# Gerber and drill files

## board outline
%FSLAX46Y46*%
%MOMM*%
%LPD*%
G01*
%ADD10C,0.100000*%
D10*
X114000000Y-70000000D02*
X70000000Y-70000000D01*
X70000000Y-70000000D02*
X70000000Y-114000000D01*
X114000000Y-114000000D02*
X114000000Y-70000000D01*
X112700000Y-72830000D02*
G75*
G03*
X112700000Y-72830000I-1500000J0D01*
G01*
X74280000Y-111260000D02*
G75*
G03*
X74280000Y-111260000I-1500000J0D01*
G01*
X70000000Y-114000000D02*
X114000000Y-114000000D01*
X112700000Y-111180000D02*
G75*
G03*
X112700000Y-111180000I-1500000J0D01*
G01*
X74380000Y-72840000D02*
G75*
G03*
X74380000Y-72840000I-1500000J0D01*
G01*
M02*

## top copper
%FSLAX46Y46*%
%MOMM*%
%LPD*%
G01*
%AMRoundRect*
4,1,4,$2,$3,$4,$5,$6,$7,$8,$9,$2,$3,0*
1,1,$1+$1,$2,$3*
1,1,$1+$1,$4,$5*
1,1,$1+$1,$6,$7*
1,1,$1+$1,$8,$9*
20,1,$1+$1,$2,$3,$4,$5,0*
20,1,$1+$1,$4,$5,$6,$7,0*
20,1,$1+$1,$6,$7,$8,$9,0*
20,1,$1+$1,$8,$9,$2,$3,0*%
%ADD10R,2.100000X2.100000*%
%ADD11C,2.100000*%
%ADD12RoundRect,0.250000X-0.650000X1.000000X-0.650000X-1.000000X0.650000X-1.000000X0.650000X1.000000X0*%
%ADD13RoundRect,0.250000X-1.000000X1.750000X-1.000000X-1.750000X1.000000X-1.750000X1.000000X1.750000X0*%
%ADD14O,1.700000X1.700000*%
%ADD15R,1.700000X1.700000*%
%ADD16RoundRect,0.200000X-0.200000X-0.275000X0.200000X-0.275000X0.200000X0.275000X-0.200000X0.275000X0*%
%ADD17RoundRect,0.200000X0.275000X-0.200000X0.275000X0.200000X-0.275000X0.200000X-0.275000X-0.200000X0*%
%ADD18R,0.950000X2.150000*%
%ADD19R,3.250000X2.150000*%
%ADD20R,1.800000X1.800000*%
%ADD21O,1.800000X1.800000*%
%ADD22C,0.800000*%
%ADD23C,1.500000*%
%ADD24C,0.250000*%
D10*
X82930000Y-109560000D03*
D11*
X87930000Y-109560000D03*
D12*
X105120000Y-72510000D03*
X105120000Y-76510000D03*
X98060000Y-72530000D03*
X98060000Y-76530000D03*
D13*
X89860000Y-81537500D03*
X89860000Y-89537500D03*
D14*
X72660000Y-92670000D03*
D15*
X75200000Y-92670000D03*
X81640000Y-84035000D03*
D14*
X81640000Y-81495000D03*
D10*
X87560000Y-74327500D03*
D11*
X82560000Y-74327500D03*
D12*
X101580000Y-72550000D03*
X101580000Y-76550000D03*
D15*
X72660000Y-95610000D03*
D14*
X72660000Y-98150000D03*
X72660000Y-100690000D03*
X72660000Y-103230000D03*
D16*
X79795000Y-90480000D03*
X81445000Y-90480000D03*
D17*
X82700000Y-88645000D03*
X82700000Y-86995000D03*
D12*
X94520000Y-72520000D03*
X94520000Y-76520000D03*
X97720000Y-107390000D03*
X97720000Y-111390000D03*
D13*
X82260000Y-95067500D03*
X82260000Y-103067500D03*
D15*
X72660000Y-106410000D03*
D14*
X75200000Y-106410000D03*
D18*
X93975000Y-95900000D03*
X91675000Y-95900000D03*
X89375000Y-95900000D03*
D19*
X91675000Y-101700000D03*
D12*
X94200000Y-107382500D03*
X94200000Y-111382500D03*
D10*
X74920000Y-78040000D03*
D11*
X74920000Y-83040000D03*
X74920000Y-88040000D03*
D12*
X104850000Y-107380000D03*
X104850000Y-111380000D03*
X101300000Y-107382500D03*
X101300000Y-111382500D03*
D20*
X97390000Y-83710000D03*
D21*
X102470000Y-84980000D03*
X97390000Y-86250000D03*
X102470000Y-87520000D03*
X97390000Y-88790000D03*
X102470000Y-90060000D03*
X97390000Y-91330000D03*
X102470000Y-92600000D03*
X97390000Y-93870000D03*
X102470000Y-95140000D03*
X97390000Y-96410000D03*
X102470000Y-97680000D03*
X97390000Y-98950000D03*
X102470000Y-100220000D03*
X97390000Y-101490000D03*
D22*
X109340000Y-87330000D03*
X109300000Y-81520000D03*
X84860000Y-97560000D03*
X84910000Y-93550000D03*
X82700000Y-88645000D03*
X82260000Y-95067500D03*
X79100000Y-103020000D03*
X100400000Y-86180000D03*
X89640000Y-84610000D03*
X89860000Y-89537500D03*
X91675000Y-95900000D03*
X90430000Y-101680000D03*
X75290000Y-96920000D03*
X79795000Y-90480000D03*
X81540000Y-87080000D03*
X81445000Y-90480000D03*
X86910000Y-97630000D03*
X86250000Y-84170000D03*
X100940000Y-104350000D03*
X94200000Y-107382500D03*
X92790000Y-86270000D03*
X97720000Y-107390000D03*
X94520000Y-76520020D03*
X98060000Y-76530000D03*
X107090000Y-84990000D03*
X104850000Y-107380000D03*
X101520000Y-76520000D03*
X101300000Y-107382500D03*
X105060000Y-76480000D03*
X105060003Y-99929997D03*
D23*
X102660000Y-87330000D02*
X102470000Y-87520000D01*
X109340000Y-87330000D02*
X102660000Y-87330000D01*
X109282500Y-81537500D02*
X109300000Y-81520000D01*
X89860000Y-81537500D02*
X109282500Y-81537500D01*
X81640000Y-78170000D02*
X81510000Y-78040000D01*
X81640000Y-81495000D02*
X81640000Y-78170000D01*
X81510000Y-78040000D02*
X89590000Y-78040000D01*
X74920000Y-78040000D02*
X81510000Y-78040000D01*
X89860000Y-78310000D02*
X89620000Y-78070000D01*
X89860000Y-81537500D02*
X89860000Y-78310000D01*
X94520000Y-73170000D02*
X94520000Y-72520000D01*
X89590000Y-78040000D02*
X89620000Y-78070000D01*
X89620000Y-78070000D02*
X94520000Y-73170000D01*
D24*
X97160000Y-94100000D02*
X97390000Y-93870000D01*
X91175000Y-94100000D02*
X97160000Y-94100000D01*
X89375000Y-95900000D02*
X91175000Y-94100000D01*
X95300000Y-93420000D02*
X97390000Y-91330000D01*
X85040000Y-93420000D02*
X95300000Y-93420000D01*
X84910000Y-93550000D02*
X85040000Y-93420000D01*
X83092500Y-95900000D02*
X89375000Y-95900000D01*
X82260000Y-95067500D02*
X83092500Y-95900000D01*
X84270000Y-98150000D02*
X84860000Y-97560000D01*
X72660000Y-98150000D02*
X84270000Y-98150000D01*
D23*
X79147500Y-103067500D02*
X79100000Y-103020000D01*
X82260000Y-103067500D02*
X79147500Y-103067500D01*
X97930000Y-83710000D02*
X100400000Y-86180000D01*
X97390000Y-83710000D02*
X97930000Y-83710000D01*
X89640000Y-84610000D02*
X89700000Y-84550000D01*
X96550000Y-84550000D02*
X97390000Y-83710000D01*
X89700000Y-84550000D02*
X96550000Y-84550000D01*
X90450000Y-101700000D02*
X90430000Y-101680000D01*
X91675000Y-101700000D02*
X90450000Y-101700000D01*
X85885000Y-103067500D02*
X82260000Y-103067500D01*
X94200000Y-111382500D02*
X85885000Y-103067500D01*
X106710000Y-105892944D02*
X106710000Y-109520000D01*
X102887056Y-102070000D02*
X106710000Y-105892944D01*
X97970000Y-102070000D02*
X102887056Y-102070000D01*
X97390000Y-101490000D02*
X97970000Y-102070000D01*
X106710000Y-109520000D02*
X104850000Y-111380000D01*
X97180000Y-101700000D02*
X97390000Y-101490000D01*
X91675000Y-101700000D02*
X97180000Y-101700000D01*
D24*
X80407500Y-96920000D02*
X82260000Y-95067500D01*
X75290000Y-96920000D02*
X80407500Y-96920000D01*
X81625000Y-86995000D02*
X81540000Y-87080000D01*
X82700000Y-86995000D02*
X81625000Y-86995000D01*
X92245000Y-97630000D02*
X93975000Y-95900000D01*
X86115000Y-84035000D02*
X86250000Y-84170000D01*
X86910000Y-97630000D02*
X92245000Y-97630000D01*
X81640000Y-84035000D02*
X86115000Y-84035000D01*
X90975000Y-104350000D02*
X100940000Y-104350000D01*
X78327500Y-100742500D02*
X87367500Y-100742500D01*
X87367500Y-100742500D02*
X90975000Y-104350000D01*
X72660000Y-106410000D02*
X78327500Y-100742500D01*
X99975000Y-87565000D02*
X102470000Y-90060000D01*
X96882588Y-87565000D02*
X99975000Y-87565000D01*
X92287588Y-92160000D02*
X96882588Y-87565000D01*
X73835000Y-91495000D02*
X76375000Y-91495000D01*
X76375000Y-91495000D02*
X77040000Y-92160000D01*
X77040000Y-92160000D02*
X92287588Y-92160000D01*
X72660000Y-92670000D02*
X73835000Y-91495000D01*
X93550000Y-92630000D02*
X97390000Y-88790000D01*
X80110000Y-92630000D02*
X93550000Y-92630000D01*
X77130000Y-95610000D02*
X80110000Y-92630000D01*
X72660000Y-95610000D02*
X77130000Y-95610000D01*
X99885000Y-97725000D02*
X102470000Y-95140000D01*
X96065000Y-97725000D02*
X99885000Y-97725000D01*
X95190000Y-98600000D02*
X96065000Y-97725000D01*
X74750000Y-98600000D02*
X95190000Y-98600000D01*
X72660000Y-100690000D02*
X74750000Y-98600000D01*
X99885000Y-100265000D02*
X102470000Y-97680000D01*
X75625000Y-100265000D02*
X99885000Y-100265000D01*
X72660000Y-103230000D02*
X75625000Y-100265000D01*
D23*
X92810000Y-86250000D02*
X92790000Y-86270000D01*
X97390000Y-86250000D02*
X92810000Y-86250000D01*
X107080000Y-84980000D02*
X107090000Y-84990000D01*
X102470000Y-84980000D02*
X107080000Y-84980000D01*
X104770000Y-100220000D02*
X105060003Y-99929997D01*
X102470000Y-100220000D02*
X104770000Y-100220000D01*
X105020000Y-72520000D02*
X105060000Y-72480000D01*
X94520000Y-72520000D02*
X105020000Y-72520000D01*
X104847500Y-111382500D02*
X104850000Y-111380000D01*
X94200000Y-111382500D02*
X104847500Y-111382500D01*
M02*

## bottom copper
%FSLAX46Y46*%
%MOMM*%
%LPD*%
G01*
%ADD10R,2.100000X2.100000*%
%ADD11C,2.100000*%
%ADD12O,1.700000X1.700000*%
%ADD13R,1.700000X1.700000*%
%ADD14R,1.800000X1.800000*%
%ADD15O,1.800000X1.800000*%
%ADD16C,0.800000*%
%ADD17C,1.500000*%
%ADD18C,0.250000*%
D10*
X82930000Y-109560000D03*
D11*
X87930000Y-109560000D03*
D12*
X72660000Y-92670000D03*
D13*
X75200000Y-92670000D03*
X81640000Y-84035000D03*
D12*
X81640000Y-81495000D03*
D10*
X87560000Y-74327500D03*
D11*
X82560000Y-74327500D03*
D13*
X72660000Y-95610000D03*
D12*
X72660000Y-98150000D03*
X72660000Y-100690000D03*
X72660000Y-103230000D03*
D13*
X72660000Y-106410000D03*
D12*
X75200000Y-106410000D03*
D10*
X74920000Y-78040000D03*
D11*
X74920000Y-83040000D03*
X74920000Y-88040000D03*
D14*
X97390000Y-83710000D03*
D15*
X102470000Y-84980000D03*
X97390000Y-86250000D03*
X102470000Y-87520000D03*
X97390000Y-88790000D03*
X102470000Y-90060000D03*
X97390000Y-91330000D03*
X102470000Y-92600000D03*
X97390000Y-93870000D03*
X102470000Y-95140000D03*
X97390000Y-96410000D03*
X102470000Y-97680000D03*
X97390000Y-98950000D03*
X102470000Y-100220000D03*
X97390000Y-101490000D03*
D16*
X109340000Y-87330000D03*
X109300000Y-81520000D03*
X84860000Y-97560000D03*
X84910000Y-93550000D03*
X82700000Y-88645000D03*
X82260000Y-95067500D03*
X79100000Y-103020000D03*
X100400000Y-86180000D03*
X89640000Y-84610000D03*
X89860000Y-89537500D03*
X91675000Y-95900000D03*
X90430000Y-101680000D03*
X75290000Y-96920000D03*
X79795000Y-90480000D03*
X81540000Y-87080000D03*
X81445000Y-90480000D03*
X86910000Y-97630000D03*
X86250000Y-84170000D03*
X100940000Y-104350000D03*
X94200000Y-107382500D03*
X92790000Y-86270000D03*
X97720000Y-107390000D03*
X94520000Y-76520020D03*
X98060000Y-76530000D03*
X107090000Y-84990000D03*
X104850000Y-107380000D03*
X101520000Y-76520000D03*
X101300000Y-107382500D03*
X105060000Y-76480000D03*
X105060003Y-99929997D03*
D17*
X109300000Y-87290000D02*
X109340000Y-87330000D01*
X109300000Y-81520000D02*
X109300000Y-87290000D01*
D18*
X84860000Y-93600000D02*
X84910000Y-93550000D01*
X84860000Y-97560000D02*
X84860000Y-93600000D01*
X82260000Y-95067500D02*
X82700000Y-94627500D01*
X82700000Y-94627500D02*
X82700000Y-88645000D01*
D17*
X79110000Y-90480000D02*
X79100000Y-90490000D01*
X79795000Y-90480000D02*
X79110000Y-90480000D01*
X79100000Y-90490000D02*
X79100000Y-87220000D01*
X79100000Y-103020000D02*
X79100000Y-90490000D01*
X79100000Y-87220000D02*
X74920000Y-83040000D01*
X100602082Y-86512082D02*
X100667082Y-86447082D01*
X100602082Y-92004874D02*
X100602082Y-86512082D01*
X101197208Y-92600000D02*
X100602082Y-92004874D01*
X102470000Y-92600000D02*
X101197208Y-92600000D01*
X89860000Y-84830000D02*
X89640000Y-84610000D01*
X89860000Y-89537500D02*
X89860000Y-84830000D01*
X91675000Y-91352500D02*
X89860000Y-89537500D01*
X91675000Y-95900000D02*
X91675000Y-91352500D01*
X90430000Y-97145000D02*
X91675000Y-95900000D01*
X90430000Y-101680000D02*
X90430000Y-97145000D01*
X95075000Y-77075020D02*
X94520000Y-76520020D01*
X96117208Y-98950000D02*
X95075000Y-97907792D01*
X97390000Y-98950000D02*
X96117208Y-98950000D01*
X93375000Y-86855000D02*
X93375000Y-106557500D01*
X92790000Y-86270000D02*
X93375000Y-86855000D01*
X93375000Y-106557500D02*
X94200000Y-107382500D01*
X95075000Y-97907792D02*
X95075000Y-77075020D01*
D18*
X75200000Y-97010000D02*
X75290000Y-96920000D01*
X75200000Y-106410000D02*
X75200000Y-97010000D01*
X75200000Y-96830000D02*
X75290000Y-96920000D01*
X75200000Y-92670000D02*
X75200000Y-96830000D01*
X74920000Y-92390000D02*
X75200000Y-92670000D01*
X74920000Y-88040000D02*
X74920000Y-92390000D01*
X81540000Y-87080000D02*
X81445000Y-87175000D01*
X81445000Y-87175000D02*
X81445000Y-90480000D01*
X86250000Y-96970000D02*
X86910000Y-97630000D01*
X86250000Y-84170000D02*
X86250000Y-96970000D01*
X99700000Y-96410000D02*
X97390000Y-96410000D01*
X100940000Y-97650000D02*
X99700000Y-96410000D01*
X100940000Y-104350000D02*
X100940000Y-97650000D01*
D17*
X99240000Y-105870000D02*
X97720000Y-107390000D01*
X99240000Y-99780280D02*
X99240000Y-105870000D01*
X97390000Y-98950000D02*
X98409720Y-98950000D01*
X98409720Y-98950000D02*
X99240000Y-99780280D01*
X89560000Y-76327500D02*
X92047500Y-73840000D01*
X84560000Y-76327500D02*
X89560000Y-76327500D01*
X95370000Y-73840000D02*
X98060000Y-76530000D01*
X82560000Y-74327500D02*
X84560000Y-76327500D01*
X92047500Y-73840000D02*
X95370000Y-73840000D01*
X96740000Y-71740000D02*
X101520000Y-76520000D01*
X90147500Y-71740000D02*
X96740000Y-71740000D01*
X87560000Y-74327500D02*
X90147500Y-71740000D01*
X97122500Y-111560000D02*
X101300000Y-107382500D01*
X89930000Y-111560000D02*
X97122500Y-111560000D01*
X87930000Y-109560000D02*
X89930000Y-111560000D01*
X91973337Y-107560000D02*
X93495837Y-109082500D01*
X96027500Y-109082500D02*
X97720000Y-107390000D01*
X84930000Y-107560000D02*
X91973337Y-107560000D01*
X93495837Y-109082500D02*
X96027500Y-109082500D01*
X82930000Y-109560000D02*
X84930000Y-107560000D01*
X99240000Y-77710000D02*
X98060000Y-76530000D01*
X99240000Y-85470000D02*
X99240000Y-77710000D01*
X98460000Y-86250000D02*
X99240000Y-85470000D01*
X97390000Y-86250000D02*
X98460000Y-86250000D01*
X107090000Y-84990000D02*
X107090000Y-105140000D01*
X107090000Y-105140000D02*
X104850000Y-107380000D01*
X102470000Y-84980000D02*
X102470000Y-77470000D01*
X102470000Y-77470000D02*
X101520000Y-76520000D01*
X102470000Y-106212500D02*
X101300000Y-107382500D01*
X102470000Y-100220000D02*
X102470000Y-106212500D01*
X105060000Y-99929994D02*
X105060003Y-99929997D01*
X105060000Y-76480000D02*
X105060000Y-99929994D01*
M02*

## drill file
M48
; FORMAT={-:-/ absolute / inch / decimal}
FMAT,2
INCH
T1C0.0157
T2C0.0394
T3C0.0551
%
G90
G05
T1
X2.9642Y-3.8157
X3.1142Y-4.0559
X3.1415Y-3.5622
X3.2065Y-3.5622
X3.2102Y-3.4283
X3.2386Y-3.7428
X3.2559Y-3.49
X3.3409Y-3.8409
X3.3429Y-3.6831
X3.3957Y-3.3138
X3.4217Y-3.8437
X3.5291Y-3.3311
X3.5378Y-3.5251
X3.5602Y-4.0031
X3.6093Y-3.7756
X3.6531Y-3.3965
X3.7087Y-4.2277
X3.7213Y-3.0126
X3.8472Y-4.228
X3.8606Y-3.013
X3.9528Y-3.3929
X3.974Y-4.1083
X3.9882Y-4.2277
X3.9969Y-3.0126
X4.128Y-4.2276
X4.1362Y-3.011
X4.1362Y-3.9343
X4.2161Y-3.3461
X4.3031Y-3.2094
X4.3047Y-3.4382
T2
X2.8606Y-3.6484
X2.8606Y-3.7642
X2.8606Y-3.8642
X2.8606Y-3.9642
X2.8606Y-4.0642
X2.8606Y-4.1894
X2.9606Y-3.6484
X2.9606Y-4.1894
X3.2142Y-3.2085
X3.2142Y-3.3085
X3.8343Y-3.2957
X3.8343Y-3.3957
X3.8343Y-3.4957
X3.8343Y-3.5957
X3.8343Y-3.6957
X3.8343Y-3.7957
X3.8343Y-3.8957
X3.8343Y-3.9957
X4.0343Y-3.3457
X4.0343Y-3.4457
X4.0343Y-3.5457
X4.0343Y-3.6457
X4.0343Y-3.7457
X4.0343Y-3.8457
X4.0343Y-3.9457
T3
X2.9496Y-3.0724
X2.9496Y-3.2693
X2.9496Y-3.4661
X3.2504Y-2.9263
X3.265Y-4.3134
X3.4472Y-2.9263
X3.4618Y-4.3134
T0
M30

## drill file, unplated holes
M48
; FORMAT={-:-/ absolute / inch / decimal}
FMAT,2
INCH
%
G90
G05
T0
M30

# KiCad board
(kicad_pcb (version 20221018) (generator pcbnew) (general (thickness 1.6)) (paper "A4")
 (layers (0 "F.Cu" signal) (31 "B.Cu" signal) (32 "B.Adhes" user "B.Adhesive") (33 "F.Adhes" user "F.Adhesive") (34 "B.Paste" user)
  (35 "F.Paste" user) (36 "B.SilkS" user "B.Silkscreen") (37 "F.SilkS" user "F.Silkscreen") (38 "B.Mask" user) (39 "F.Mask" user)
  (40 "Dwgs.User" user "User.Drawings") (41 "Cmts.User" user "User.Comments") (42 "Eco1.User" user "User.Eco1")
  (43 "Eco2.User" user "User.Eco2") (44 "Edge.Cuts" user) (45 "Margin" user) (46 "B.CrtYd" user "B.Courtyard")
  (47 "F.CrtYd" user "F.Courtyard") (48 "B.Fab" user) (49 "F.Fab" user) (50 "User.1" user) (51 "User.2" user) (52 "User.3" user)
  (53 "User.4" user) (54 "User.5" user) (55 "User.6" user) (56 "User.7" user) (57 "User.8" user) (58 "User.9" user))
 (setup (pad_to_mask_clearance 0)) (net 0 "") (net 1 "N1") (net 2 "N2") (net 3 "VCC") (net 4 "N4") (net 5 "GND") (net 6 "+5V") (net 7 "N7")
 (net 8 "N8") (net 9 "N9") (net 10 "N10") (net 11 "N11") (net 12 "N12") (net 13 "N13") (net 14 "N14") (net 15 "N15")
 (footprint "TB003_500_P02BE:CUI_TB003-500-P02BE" (layer "F.Cu") (at 82.93 109.56)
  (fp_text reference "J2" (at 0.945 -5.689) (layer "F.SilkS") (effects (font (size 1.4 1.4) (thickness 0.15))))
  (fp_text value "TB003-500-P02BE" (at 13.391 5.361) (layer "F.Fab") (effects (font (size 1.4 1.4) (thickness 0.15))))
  (pad "1" thru_hole rect (at 0 0) (size 2.1 2.1) (drill 1.4) (layers "*.Cu" "*.Mask") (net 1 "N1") (solder_mask_margin 0.102))
  (pad "2" thru_hole circle (at 5 0) (size 2.1 2.1) (drill 1.4) (layers "*.Cu" "*.Mask") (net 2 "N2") (solder_mask_margin 0.102)))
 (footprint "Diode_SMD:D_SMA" (layer "F.Cu") (at 105.12 74.51 -90)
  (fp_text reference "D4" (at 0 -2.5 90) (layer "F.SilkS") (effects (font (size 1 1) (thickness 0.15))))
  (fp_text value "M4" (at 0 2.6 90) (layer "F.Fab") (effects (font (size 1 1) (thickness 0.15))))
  (pad "1" smd roundrect (at -2 0 270) (size 2.5 1.8) (layers "F.Cu" "F.Paste" "F.Mask") (roundrect_rratio 0.1388888889) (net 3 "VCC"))
  (pad "2" smd roundrect (at 2 0 270) (size 2.5 1.8) (layers "F.Cu" "F.Paste" "F.Mask") (roundrect_rratio 0.1388888889) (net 2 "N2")))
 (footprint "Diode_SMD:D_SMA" (layer "F.Cu") (at 98.06 74.53 -90)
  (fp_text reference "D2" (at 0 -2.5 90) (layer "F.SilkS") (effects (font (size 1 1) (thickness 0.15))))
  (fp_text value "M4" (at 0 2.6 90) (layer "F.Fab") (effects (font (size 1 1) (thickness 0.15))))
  (pad "1" smd roundrect (at -2 0 270) (size 2.5 1.8) (layers "F.Cu" "F.Paste" "F.Mask") (roundrect_rratio 0.1388888889) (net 3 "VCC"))
  (pad "2" smd roundrect (at 2 0 270) (size 2.5 1.8) (layers "F.Cu" "F.Paste" "F.Mask") (roundrect_rratio 0.1388888889) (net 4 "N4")))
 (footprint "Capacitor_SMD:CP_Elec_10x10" (layer "F.Cu") (at 89.86 85.5375 -90)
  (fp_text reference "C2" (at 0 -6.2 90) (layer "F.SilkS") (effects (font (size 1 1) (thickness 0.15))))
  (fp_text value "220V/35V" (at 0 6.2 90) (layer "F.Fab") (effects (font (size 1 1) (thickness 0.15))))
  (pad "1" smd roundrect (at -4 0 270) (size 4 2.5) (layers "F.Cu" "F.Paste" "F.Mask") (roundrect_rratio 0.1) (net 3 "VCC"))
  (pad "2" smd roundrect (at 4 0 270) (size 4 2.5) (layers "F.Cu" "F.Paste" "F.Mask") (roundrect_rratio 0.1) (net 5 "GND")))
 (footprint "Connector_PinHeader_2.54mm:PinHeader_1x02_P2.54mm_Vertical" (layer "F.Cu") (at 75.2 92.67 -90)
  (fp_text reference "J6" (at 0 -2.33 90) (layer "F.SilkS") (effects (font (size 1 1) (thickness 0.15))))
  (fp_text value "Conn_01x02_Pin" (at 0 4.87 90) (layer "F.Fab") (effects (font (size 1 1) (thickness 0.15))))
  (pad "1" thru_hole rect (at 0 0 270) (size 1.7 1.7) (drill 1) (layers "*.Cu" "*.Mask") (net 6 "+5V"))
  (pad "2" thru_hole oval (at 0 2.54 270) (size 1.7 1.7) (drill 1) (layers "*.Cu" "*.Mask") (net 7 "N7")))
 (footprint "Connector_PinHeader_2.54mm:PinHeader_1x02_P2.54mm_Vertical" (layer "F.Cu") (at 81.64 84.035 180)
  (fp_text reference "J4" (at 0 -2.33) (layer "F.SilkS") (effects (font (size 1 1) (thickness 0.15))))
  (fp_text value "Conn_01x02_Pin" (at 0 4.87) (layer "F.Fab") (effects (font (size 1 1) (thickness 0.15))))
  (pad "1" thru_hole rect (at 0 0 180) (size 1.7 1.7) (drill 1) (layers "*.Cu" "*.Mask") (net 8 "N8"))
  (pad "2" thru_hole oval (at 0 2.54 180) (size 1.7 1.7) (drill 1) (layers "*.Cu" "*.Mask") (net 3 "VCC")))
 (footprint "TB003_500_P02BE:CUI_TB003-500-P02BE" (layer "F.Cu") (at 87.56 74.3275 180)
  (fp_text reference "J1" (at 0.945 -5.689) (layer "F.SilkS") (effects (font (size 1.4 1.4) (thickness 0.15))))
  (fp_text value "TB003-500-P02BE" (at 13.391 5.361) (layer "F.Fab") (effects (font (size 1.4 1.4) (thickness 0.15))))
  (pad "1" thru_hole rect (at 0 0 180) (size 2.1 2.1) (drill 1.4) (layers "*.Cu" "*.Mask") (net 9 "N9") (solder_mask_margin 0.102))
  (pad "2" thru_hole circle (at 5 0 180) (size 2.1 2.1) (drill 1.4) (layers "*.Cu" "*.Mask") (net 4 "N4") (solder_mask_margin 0.102)))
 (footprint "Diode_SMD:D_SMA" (layer "F.Cu") (at 101.58 74.55 -90)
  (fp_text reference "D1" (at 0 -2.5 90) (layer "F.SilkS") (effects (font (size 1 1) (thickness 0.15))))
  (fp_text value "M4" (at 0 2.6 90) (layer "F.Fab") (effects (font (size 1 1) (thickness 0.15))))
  (pad "1" smd roundrect (at -2 0 270) (size 2.5 1.8) (layers "F.Cu" "F.Paste" "F.Mask") (roundrect_rratio 0.1388888889) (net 3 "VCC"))
  (pad "2" smd roundrect (at 2 0 270) (size 2.5 1.8) (layers "F.Cu" "F.Paste" "F.Mask") (roundrect_rratio 0.1388888889) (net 9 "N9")))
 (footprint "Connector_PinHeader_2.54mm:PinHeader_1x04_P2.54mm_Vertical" (layer "F.Cu") (at 72.66 95.61)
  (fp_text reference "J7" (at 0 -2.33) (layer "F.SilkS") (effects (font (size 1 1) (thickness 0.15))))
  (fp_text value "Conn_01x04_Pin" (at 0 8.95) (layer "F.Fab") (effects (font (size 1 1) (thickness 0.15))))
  (pad "1" thru_hole rect (at 0 0) (size 1.7 1.7) (drill 1) (layers "*.Cu" "*.Mask") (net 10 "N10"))
  (pad "2" thru_hole oval (at 0 2.54) (size 1.7 1.7) (drill 1) (layers "*.Cu" "*.Mask") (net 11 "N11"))
  (pad "3" thru_hole oval (at 0 5.08) (size 1.7 1.7) (drill 1) (layers "*.Cu" "*.Mask") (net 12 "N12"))
  (pad "4" thru_hole oval (at 0 7.62) (size 1.7 1.7) (drill 1) (layers "*.Cu" "*.Mask") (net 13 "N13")))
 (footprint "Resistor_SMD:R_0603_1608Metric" (layer "F.Cu") (at 80.62 90.48)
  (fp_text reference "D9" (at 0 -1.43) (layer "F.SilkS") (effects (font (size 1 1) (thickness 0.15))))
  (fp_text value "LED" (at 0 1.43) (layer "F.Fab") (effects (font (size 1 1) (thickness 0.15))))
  (pad "1" smd roundrect (at -0.825 0) (size 0.8 0.95) (layers "F.Cu" "F.Paste" "F.Mask") (roundrect_rratio 0.25) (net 5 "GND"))
  (pad "2" smd roundrect (at 0.825 0) (size 0.8 0.95) (layers "F.Cu" "F.Paste" "F.Mask") (roundrect_rratio 0.25) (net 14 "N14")))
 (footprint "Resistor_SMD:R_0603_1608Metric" (layer "F.Cu") (at 82.7 87.82 90)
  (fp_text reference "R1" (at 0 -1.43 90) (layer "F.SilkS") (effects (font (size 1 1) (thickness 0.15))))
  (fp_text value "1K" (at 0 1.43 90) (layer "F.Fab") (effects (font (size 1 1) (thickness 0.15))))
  (pad "1" smd roundrect (at -0.825 0 90) (size 0.8 0.95) (layers "F.Cu" "F.Paste" "F.Mask") (roundrect_rratio 0.25) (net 6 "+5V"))
  (pad "2" smd roundrect (at 0.825 0 90) (size 0.8 0.95) (layers "F.Cu" "F.Paste" "F.Mask") (roundrect_rratio 0.25) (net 14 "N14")))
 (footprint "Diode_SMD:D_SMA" (layer "F.Cu") (at 94.52 74.52 -90)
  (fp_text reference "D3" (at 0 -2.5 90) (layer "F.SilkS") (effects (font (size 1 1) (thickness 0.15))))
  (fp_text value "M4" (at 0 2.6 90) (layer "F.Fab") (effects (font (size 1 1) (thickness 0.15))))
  (pad "1" smd roundrect (at -2 0 270) (size 2.5 1.8) (layers "F.Cu" "F.Paste" "F.Mask") (roundrect_rratio 0.1388888889) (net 3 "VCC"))
  (pad "2" smd roundrect (at 2 0 270) (size 2.5 1.8) (layers "F.Cu" "F.Paste" "F.Mask") (roundrect_rratio 0.1388888889) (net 1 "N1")))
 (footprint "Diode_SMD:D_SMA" (layer "F.Cu") (at 97.72 109.39 -90)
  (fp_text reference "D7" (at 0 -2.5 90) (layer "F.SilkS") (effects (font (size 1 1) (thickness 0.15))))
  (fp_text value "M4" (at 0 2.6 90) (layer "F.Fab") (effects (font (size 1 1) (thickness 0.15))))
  (pad "1" smd roundrect (at -2 0 270) (size 2.5 1.8) (layers "F.Cu" "F.Paste" "F.Mask") (roundrect_rratio 0.1388888889) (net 1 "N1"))
  (pad "2" smd roundrect (at 2 0 270) (size 2.5 1.8) (layers "F.Cu" "F.Paste" "F.Mask") (roundrect_rratio 0.1388888889) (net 5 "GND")))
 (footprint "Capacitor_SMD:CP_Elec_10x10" (layer "F.Cu") (at 82.26 99.0675 -90)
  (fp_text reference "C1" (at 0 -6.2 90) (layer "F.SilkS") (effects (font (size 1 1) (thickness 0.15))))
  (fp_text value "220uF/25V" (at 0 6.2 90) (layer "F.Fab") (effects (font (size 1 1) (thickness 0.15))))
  (pad "1" smd roundrect (at -4 0 270) (size 4 2.5) (layers "F.Cu" "F.Paste" "F.Mask") (roundrect_rratio 0.1) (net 6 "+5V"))
  (pad "2" smd roundrect (at 4 0 270) (size 4 2.5) (layers "F.Cu" "F.Paste" "F.Mask") (roundrect_rratio 0.1) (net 5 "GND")))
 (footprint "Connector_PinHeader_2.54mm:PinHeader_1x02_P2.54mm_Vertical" (layer "F.Cu") (at 72.66 106.41 90)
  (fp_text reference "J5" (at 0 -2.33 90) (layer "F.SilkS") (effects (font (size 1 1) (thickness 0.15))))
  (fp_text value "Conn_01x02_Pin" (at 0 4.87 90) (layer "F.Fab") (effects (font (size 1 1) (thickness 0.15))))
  (pad "1" thru_hole rect (at 0 0 90) (size 1.7 1.7) (drill 1) (layers "*.Cu" "*.Mask") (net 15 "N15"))
  (pad "2" thru_hole oval (at 0 2.54 90) (size 1.7 1.7) (drill 1) (layers "*.Cu" "*.Mask") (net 6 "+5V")))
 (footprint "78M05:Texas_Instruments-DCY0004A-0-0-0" (layer "F.Cu") (at 91.675 98.8 180)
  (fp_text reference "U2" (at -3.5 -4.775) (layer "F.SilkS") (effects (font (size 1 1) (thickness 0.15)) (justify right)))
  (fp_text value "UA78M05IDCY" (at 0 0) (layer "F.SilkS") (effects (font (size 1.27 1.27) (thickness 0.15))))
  (pad "1" smd rect (at -2.3 2.9 180) (size 0.95 2.15) (layers "F.Cu" "F.Paste" "F.Mask") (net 8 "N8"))
  (pad "2" smd rect (at 0 2.9 180) (size 0.95 2.15) (layers "F.Cu" "F.Paste" "F.Mask") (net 5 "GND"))
  (pad "3" smd rect (at 2.3 2.9 180) (size 0.95 2.15) (layers "F.Cu" "F.Paste" "F.Mask") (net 6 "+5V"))
  (pad "4" smd rect (at 0 -2.9 180) (size 3.25 2.15) (layers "F.Cu" "F.Paste" "F.Mask") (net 5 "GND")))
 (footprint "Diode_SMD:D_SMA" (layer "F.Cu") (at 94.2 109.3825 -90)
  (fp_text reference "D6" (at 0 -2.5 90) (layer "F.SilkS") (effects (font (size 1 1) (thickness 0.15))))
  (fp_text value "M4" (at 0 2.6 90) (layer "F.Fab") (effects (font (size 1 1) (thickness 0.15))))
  (pad "1" smd roundrect (at -2 0 270) (size 2.5 1.8) (layers "F.Cu" "F.Paste" "F.Mask") (roundrect_rratio 0.1388888889) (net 4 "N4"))
  (pad "2" smd roundrect (at 2 0 270) (size 2.5 1.8) (layers "F.Cu" "F.Paste" "F.Mask") (roundrect_rratio 0.1388888889) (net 5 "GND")))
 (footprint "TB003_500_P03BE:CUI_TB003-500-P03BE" (layer "F.Cu") (at 74.92 78.04 -90)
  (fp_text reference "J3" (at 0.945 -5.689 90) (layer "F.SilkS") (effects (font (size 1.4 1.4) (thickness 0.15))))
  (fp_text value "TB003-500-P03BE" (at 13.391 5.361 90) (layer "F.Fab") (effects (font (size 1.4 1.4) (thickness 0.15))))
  (pad "1" thru_hole rect (at 0 0 270) (size 2.1 2.1) (drill 1.4) (layers "*.Cu" "*.Mask") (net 3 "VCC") (solder_mask_margin 0.102))
  (pad "2" thru_hole circle (at 5 0 270) (size 2.1 2.1) (drill 1.4) (layers "*.Cu" "*.Mask") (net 5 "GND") (solder_mask_margin 0.102))
  (pad "3" thru_hole circle (at 10 0 270) (size 2.1 2.1) (drill 1.4) (layers "*.Cu" "*.Mask") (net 6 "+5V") (solder_mask_margin 0.102)))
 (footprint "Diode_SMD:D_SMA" (layer "F.Cu") (at 104.85 109.38 -90)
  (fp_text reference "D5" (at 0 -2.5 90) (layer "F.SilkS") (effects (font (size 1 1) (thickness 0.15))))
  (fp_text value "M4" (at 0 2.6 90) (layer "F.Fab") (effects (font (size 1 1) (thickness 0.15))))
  (pad "1" smd roundrect (at -2 0 270) (size 2.5 1.8) (layers "F.Cu" "F.Paste" "F.Mask") (roundrect_rratio 0.1388888889) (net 9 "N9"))
  (pad "2" smd roundrect (at 2 0 270) (size 2.5 1.8) (layers "F.Cu" "F.Paste" "F.Mask") (roundrect_rratio 0.1388888889) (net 5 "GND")))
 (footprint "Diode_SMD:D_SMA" (layer "F.Cu") (at 101.3 109.3825 -90)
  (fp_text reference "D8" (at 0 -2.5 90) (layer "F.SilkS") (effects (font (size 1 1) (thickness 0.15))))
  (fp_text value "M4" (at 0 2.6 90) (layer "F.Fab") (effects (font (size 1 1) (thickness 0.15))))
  (pad "1" smd roundrect (at -2 0 270) (size 2.5 1.8) (layers "F.Cu" "F.Paste" "F.Mask") (roundrect_rratio 0.1388888889) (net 2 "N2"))
  (pad "2" smd roundrect (at 2 0 270) (size 2.5 1.8) (layers "F.Cu" "F.Paste" "F.Mask") (roundrect_rratio 0.1388888889) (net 5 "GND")))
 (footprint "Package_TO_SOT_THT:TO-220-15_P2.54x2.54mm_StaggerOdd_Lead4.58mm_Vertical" (layer "F.Cu") (at 97.39 83.71 -90)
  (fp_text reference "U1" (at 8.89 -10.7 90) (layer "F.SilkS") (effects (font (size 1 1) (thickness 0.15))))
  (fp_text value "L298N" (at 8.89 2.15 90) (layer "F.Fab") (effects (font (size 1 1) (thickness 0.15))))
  (pad "1" thru_hole rect (at 0 0 270) (size 1.8 1.8) (drill 1) (layers "*.Cu" "*.Mask") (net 5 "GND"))
  (pad "2" thru_hole oval (at 1.27 -5.08 270) (size 1.8 1.8) (drill 1) (layers "*.Cu" "*.Mask") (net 9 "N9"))
  (pad "3" thru_hole oval (at 2.54 0 270) (size 1.8 1.8) (drill 1) (layers "*.Cu" "*.Mask") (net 4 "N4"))
  (pad "4" thru_hole oval (at 3.81 -5.08 270) (size 1.8 1.8) (drill 1) (layers "*.Cu" "*.Mask") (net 3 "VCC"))
  (pad "5" thru_hole oval (at 5.08 0 270) (size 1.8 1.8) (drill 1) (layers "*.Cu" "*.Mask") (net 10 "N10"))
  (pad "6" thru_hole oval (at 6.35 -5.08 270) (size 1.8 1.8) (drill 1) (layers "*.Cu" "*.Mask") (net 7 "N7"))
  (pad "7" thru_hole oval (at 7.62 0 270) (size 1.8 1.8) (drill 1) (layers "*.Cu" "*.Mask") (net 11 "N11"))
  (pad "8" thru_hole oval (at 8.89 -5.08 270) (size 1.8 1.8) (drill 1) (layers "*.Cu" "*.Mask") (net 5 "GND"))
  (pad "9" thru_hole oval (at 10.16 0 270) (size 1.8 1.8) (drill 1) (layers "*.Cu" "*.Mask") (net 6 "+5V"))
  (pad "10" thru_hole oval (at 11.43 -5.08 270) (size 1.8 1.8) (drill 1) (layers "*.Cu" "*.Mask") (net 12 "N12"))
  (pad "11" thru_hole oval (at 12.7 0 270) (size 1.8 1.8) (drill 1) (layers "*.Cu" "*.Mask") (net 15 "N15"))
  (pad "12" thru_hole oval (at 13.97 -5.08 270) (size 1.8 1.8) (drill 1) (layers "*.Cu" "*.Mask") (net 13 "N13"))
  (pad "13" thru_hole oval (at 15.24 0 270) (size 1.8 1.8) (drill 1) (layers "*.Cu" "*.Mask") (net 1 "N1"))
  (pad "14" thru_hole oval (at 16.51 -5.08 270) (size 1.8 1.8) (drill 1) (layers "*.Cu" "*.Mask") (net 2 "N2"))
  (pad "15" thru_hole oval (at 17.78 0 270) (size 1.8 1.8) (drill 1) (layers "*.Cu" "*.Mask") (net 5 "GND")))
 (gr_line (start 114 70) (end 70 70) (stroke (width 0.1) (type default)) (layer "Edge.Cuts"))
 (gr_line (start 70 70) (end 70 114) (stroke (width 0.1) (type default)) (layer "Edge.Cuts"))
 (gr_line (start 114 114) (end 114 70) (stroke (width 0.1) (type default)) (layer "Edge.Cuts"))
 (gr_circle (center 111.2 72.83) (end 112.7 72.83) (stroke (width 0.1) (type default)) (fill none) (layer "Edge.Cuts"))
 (gr_circle (center 72.78 111.26) (end 74.28 111.26) (stroke (width 0.1) (type default)) (fill none) (layer "Edge.Cuts"))
 (gr_line (start 70 114) (end 114 114) (stroke (width 0.1) (type default)) (layer "Edge.Cuts"))
 (gr_circle (center 111.2 111.18) (end 112.7 111.18) (stroke (width 0.1) (type default)) (fill none) (layer "Edge.Cuts"))
 (gr_circle (center 72.88 72.84) (end 74.38 72.84) (stroke (width 0.1) (type default)) (fill none) (layer "Edge.Cuts"))
 (segment (start 89.375 95.9) (end 91.175 94.1) (width 0.25) (layer "F.Cu") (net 6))
 (segment (start 91.175 94.1) (end 97.16 94.1) (width 0.25) (layer "F.Cu") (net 6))
 (segment (start 82.26 95.0675) (end 83.0925 95.9) (width 0.25) (layer "F.Cu") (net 6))
 (segment (start 75.29 96.92) (end 80.4075 96.92) (width 0.25) (layer "F.Cu") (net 6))
 (segment (start 80.4075 96.92) (end 82.26 95.0675) (width 0.25) (layer "F.Cu") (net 6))
 (segment (start 97.16 94.1) (end 97.39 93.87) (width 0.25) (layer "F.Cu") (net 6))
 (segment (start 83.0925 95.9) (end 89.375 95.9) (width 0.25) (layer "F.Cu") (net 6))
 (via (at 82.7 88.645) (size 0.8) (drill 0.4) (layers "F.Cu" "B.Cu") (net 6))
 (via (at 82.26 95.0675) (size 0.8) (drill 0.4) (layers "F.Cu" "B.Cu") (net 6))
 (via (at 75.29 96.92) (size 0.8) (drill 0.4) (layers "F.Cu" "B.Cu") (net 6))
 (segment (start 82.26 95.0675) (end 82.7 94.6275) (width 0.25) (layer "B.Cu") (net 6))
 (segment (start 75.2 97.01) (end 75.29 96.92) (width 0.25) (layer "B.Cu") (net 6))
 (segment (start 82.7 94.6275) (end 82.7 88.645) (width 0.25) (layer "B.Cu") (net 6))
 (segment (start 75.2 106.41) (end 75.2 97.01) (width 0.25) (layer "B.Cu") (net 6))
 (segment (start 74.92 92.39) (end 75.2 92.67) (width 0.25) (layer "B.Cu") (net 6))
 (segment (start 75.2 92.67) (end 75.2 96.83) (width 0.25) (layer "B.Cu") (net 6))
 (segment (start 75.2 96.83) (end 75.29 96.92) (width 0.25) (layer "B.Cu") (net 6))
 (segment (start 74.92 88.04) (end 74.92 92.39) (width 0.25) (layer "B.Cu") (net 6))
 (segment (start 102.887056 102.07) (end 106.71 105.892944) (width 1.5) (layer "F.Cu") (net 5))
 (segment (start 97.39 83.71) (end 97.93 83.71) (width 1.5) (layer "F.Cu") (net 5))
 (segment (start 82.26 103.0675) (end 79.1475 103.0675) (width 1.5) (layer "F.Cu") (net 5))
 (segment (start 91.675 101.7) (end 90.45 101.7) (width 1.5) (layer "F.Cu") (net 5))
 (segment (start 89.64 84.61) (end 89.7 84.55) (width 1.5) (layer "F.Cu") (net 5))
 (segment (start 90.45 101.7) (end 90.43 101.68) (width 1.5) (layer "F.Cu") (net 5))
 (segment (start 91.675 101.7) (end 97.18 101.7) (width 1.5) (layer "F.Cu") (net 5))
 (segment (start 89.7 84.55) (end 96.55 84.55) (width 1.5) (layer "F.Cu") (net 5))
 (segment (start 85.885 103.0675) (end 82.26 103.0675) (width 1.5) (layer "F.Cu") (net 5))
 (segment (start 104.8475 111.3825) (end 104.85 111.38) (width 1.5) (layer "F.Cu") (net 5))
 (segment (start 79.1475 103.0675) (end 79.1 103.02) (width 1.5) (layer "F.Cu") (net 5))
 (segment (start 94.2 111.3825) (end 104.8475 111.3825) (width 1.5) (layer "F.Cu") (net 5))
 (segment (start 106.71 109.52) (end 104.85 111.38) (width 1.5) (layer "F.Cu") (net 5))
 (segment (start 96.55 84.55) (end 97.39 83.71) (width 1.5) (layer "F.Cu") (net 5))
 (segment (start 97.97 102.07) (end 102.887056 102.07) (width 1.5) (layer "F.Cu") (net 5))
 (segment (start 97.93 83.71) (end 100.4 86.18) (width 1.5) (layer "F.Cu") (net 5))
 (segment (start 94.2 111.3825) (end 85.885 103.0675) (width 1.5) (layer "F.Cu") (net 5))
 (segment (start 97.18 101.7) (end 97.39 101.49) (width 1.5) (layer "F.Cu") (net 5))
 (segment (start 106.71 105.892944) (end 106.71 109.52) (width 1.5) (layer "F.Cu") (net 5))
 (segment (start 97.39 101.49) (end 97.97 102.07) (width 1.5) (layer "F.Cu") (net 5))
 (via (at 79.795 90.48) (size 0.8) (drill 0.4) (layers "F.Cu" "B.Cu") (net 5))
 (via (at 89.64 84.61) (size 0.8) (drill 0.4) (layers "F.Cu" "B.Cu") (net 5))
 (via (at 90.43 101.68) (size 0.8) (drill 0.4) (layers "F.Cu" "B.Cu") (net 5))
 (via (at 100.4 86.18) (size 0.8) (drill 0.4) (layers "F.Cu" "B.Cu") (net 5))
 (via (at 89.86 89.5375) (size 0.8) (drill 0.4) (layers "F.Cu" "B.Cu") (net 5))
 (via (at 91.675 95.9) (size 0.8) (drill 0.4) (layers "F.Cu" "B.Cu") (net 5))
 (via (at 79.1 103.02) (size 0.8) (drill 0.4) (layers "F.Cu" "B.Cu") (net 5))
 (segment (start 100.602082 92.004874) (end 100.602082 86.512082) (width 1.5) (layer "B.Cu") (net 5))
 (segment (start 79.795 90.48) (end 79.11 90.48) (width 1.5) (layer "B.Cu") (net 5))
 (segment (start 90.43 97.145) (end 91.675 95.9) (width 1.5) (layer "B.Cu") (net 5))
 (segment (start 79.1 90.49) (end 79.1 87.22) (width 1.5) (layer "B.Cu") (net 5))
 (segment (start 89.86 84.83) (end 89.64 84.61) (width 1.5) (layer "B.Cu") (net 5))
 (segment (start 102.47 92.6) (end 101.197208 92.6) (width 1.5) (layer "B.Cu") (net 5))
 (segment (start 90.43 101.68) (end 90.43 97.145) (width 1.5) (layer "B.Cu") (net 5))
 (segment (start 89.86 89.5375) (end 89.86 84.83) (width 1.5) (layer "B.Cu") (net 5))
 (segment (start 91.675 95.9) (end 91.675 91.3525) (width 1.5) (layer "B.Cu") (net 5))
 (segment (start 79.11 90.48) (end 79.1 90.49) (width 1.5) (layer "B.Cu") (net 5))
 (segment (start 100.602082 86.512082) (end 100.667082 86.447082) (width 1.5) (layer "B.Cu") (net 5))
 (segment (start 91.675 91.3525) (end 89.86 89.5375) (width 1.5) (layer "B.Cu") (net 5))
 (segment (start 101.197208 92.6) (end 100.602082 92.004874) (width 1.5) (layer "B.Cu") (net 5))
 (segment (start 79.1 87.22) (end 74.92 83.04) (width 1.5) (layer "B.Cu") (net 5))
 (segment (start 79.1 103.02) (end 79.1 90.49) (width 1.5) (layer "B.Cu") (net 5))
 (segment (start 109.2825 81.5375) (end 109.3 81.52) (width 1.5) (layer "F.Cu") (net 3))
 (segment (start 94.52 72.52) (end 105.02 72.52) (width 1.5) (layer "F.Cu") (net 3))
 (segment (start 105.02 72.52) (end 105.06 72.48) (width 1.5) (layer "F.Cu") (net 3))
 (segment (start 109.34 87.33) (end 102.66 87.33) (width 1.5) (layer "F.Cu") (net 3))
 (segment (start 81.51 78.04) (end 89.59 78.04) (width 1.5) (layer "F.Cu") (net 3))
 (segment (start 89.86 81.5375) (end 89.86 78.31) (width 1.5) (layer "F.Cu") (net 3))
 (segment (start 81.64 81.495) (end 81.64 78.17) (width 1.5) (layer "F.Cu") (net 3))
 (segment (start 89.62 78.07) (end 94.52 73.17) (width 1.5) (layer "F.Cu") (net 3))
 (segment (start 94.52 73.17) (end 94.52 72.52) (width 1.5) (layer "F.Cu") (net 3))
 (segment (start 89.59 78.04) (end 89.62 78.07) (width 1.5) (layer "F.Cu") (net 3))
 (segment (start 102.66 87.33) (end 102.47 87.52) (width 1.5) (layer "F.Cu") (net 3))
 (segment (start 74.92 78.04) (end 81.51 78.04) (width 1.5) (layer "F.Cu") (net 3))
 (segment (start 89.86 78.31) (end 89.62 78.07) (width 1.5) (layer "F.Cu") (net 3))
 (segment (start 89.86 81.5375) (end 109.2825 81.5375) (width 1.5) (layer "F.Cu") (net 3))
 (segment (start 81.64 78.17) (end 81.51 78.04) (width 1.5) (layer "F.Cu") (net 3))
 (via (at 109.34 87.33) (size 0.8) (drill 0.4) (layers "F.Cu" "B.Cu") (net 3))
 (via (at 109.3 81.52) (size 0.8) (drill 0.4) (layers "F.Cu" "B.Cu") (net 3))
 (segment (start 109.3 87.29) (end 109.34 87.33) (width 1.5) (layer "B.Cu") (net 3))
 (segment (start 109.3 81.52) (end 109.3 87.29) (width 1.5) (layer "B.Cu") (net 3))
 (segment (start 102.47 84.98) (end 107.08 84.98) (width 1.5) (layer "F.Cu") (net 9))
 (segment (start 107.08 84.98) (end 107.09 84.99) (width 1.5) (layer "F.Cu") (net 9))
 (via (at 101.52 76.52) (size 0.8) (drill 0.4) (layers "F.Cu" "B.Cu") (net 9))
 (via (at 107.09 84.99) (size 0.8) (drill 0.4) (layers "F.Cu" "B.Cu") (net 9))
 (via (at 104.85 107.38) (size 0.8) (drill 0.4) (layers "F.Cu" "B.Cu") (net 9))
 (segment (start 102.47 84.98) (end 102.47 77.47) (width 1.5) (layer "B.Cu") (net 9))
 (segment (start 87.56 74.3275) (end 90.1475 71.74) (width 1.5) (layer "B.Cu") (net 9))
 (segment (start 90.1475 71.74) (end 96.74 71.74) (width 1.5) (layer "B.Cu") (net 9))
 (segment (start 102.47 77.47) (end 101.52 76.52) (width 1.5) (layer "B.Cu") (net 9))
 (segment (start 107.09 105.14) (end 104.85 107.38) (width 1.5) (layer "B.Cu") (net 9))
 (segment (start 107.09 84.99) (end 107.09 105.14) (width 1.5) (layer "B.Cu") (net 9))
 (segment (start 96.74 71.74) (end 101.52 76.52) (width 1.5) (layer "B.Cu") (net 9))
 (segment (start 92.81 86.25) (end 92.79 86.27) (width 1.5) (layer "F.Cu") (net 4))
 (segment (start 97.39 86.25) (end 92.81 86.25) (width 1.5) (layer "F.Cu") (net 4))
 (via (at 92.79 86.27) (size 0.8) (drill 0.4) (layers "F.Cu" "B.Cu") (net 4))
 (via (at 94.2 107.3825) (size 0.8) (drill 0.4) (layers "F.Cu" "B.Cu") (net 4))
 (via (at 98.06 76.53) (size 0.8) (drill 0.4) (layers "F.Cu" "B.Cu") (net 4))
 (segment (start 95.37 73.84) (end 98.06 76.53) (width 1.5) (layer "B.Cu") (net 4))
 (segment (start 99.24 77.71) (end 98.06 76.53) (width 1.5) (layer "B.Cu") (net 4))
 (segment (start 84.56 76.3275) (end 89.56 76.3275) (width 1.5) (layer "B.Cu") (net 4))
 (segment (start 98.46 86.25) (end 99.24 85.47) (width 1.5) (layer "B.Cu") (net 4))
 (segment (start 93.375 106.5575) (end 94.2 107.3825) (width 1.5) (layer "B.Cu") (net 4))
 (segment (start 92.0475 73.84) (end 95.37 73.84) (width 1.5) (layer "B.Cu") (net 4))
 (segment (start 92.79 86.27) (end 93.375 86.855) (width 1.5) (layer "B.Cu") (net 4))
 (segment (start 93.375 86.855) (end 93.375 106.5575) (width 1.5) (layer "B.Cu") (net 4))
 (segment (start 97.39 86.25) (end 98.46 86.25) (width 1.5) (layer "B.Cu") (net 4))
 (segment (start 82.56 74.3275) (end 84.56 76.3275) (width 1.5) (layer "B.Cu") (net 4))
 (segment (start 99.24 85.47) (end 99.24 77.71) (width 1.5) (layer "B.Cu") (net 4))
 (segment (start 89.56 76.3275) (end 92.0475 73.84) (width 1.5) (layer "B.Cu") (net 4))
 (via (at 97.72 107.39) (size 0.8) (drill 0.4) (layers "F.Cu" "B.Cu") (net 1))
 (via (at 94.52 76.52002) (size 0.8) (drill 0.4) (layers "F.Cu" "B.Cu") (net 1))
 (segment (start 96.117208 98.95) (end 95.075 97.907792) (width 1.5) (layer "B.Cu") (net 1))
 (segment (start 95.075 77.07502) (end 94.52 76.52002) (width 1.5) (layer "B.Cu") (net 1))
 (segment (start 99.24 105.87) (end 97.72 107.39) (width 1.5) (layer "B.Cu") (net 1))
 (segment (start 97.39 98.95) (end 98.40972 98.95) (width 1.5) (layer "B.Cu") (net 1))
 (segment (start 93.495837 109.0825) (end 96.0275 109.0825) (width 1.5) (layer "B.Cu") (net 1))
 (segment (start 82.93 109.56) (end 84.93 107.56) (width 1.5) (layer "B.Cu") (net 1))
 (segment (start 98.40972 98.95) (end 99.24 99.78028) (width 1.5) (layer "B.Cu") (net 1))
 (segment (start 91.973337 107.56) (end 93.495837 109.0825) (width 1.5) (layer "B.Cu") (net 1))
 (segment (start 84.93 107.56) (end 91.973337 107.56) (width 1.5) (layer "B.Cu") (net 1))
 (segment (start 95.075 97.907792) (end 95.075 77.07502) (width 1.5) (layer "B.Cu") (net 1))
 (segment (start 96.0275 109.0825) (end 97.72 107.39) (width 1.5) (layer "B.Cu") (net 1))
 (segment (start 97.39 98.95) (end 96.117208 98.95) (width 1.5) (layer "B.Cu") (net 1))
 (segment (start 99.24 99.78028) (end 99.24 105.87) (width 1.5) (layer "B.Cu") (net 1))
 (segment (start 102.47 100.22) (end 104.77 100.22) (width 1.5) (layer "F.Cu") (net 2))
 (segment (start 104.77 100.22) (end 105.060003 99.929997) (width 1.5) (layer "F.Cu") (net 2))
 (via (at 105.06 76.48) (size 0.8) (drill 0.4) (layers "F.Cu" "B.Cu") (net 2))
 (via (at 101.3 107.3825) (size 0.8) (drill 0.4) (layers "F.Cu" "B.Cu") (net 2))
 (via (at 105.060003 99.929997) (size 0.8) (drill 0.4) (layers "F.Cu" "B.Cu") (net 2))
 (segment (start 105.06 99.929994) (end 105.060003 99.929997) (width 1.5) (layer "B.Cu") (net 2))
 (segment (start 105.06 76.48) (end 105.06 99.929994) (width 1.5) (layer "B.Cu") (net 2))
 (segment (start 97.1225 111.56) (end 101.3 107.3825) (width 1.5) (layer "B.Cu") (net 2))
 (segment (start 89.93 111.56) (end 97.1225 111.56) (width 1.5) (layer "B.Cu") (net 2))
 (segment (start 87.93 109.56) (end 89.93 111.56) (width 1.5) (layer "B.Cu") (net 2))
 (segment (start 102.47 106.2125) (end 101.3 107.3825) (width 1.5) (layer "B.Cu") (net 2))
 (segment (start 102.47 100.22) (end 102.47 106.2125) (width 1.5) (layer "B.Cu") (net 2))
 (segment (start 86.115 84.035) (end 86.25 84.17) (width 0.25) (layer "F.Cu") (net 8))
 (segment (start 92.245 97.63) (end 93.975 95.9) (width 0.25) (layer "F.Cu") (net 8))
 (segment (start 86.91 97.63) (end 92.245 97.63) (width 0.25) (layer "F.Cu") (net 8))
 (segment (start 81.64 84.035) (end 86.115 84.035) (width 0.25) (layer "F.Cu") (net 8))
 (via (at 86.91 97.63) (size 0.8) (drill 0.4) (layers "F.Cu" "B.Cu") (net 8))
 (via (at 86.25 84.17) (size 0.8) (drill 0.4) (layers "F.Cu" "B.Cu") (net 8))
 (segment (start 86.25 84.17) (end 86.25 96.97) (width 0.25) (layer "B.Cu") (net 8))
 (segment (start 86.25 96.97) (end 86.91 97.63) (width 0.25) (layer "B.Cu") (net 8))
 (segment (start 90.975 104.35) (end 100.94 104.35) (width 0.25) (layer "F.Cu") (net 15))
 (segment (start 87.3675 100.7425) (end 90.975 104.35) (width 0.25) (layer "F.Cu") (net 15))
 (segment (start 72.66 106.41) (end 78.3275 100.7425) (width 0.25) (layer "F.Cu") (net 15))
 (segment (start 78.3275 100.7425) (end 87.3675 100.7425) (width 0.25) (layer "F.Cu") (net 15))
 (via (at 100.94 104.35) (size 0.8) (drill 0.4) (layers "F.Cu" "B.Cu") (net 15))
 (segment (start 99.7 96.41) (end 97.39 96.41) (width 0.25) (layer "B.Cu") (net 15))
 (segment (start 100.94 97.65) (end 99.7 96.41) (width 0.25) (layer "B.Cu") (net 15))
 (segment (start 100.94 104.35) (end 100.94 97.65) (width 0.25) (layer "B.Cu") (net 15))
 (segment (start 99.975 87.565) (end 102.47 90.06) (width 0.25) (layer "F.Cu") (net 7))
 (segment (start 92.287588 92.16) (end 96.882588 87.565) (width 0.25) (layer "F.Cu") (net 7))
 (segment (start 96.882588 87.565) (end 99.975 87.565) (width 0.25) (layer "F.Cu") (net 7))
 (segment (start 76.375 91.495) (end 77.04 92.16) (width 0.25) (layer "F.Cu") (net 7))
 (segment (start 73.835 91.495) (end 76.375 91.495) (width 0.25) (layer "F.Cu") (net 7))
 (segment (start 77.04 92.16) (end 92.287588 92.16) (width 0.25) (layer "F.Cu") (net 7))
 (segment (start 72.66 92.67) (end 73.835 91.495) (width 0.25) (layer "F.Cu") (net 7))
 (segment (start 93.55 92.63) (end 97.39 88.79) (width 0.25) (layer "F.Cu") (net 10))
 (segment (start 80.11 92.63) (end 93.55 92.63) (width 0.25) (layer "F.Cu") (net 10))
 (segment (start 72.66 95.61) (end 77.13 95.61) (width 0.25) (layer "F.Cu") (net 10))
 (segment (start 77.13 95.61) (end 80.11 92.63) (width 0.25) (layer "F.Cu") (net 10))
 (segment (start 85.04 93.42) (end 95.3 93.42) (width 0.25) (layer "F.Cu") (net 11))
 (segment (start 84.27 98.15) (end 84.86 97.56) (width 0.25) (layer "F.Cu") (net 11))
 (segment (start 95.3 93.42) (end 97.39 91.33) (width 0.25) (layer "F.Cu") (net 11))
 (segment (start 84.91 93.55) (end 85.04 93.42) (width 0.25) (layer "F.Cu") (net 11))
 (segment (start 72.66 98.15) (end 84.27 98.15) (width 0.25) (layer "F.Cu") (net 11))
 (via (at 84.86 97.56) (size 0.8) (drill 0.4) (layers "F.Cu" "B.Cu") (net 11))
 (via (at 84.91 93.55) (size 0.8) (drill 0.4) (layers "F.Cu" "B.Cu") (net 11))
 (segment (start 84.86 93.6) (end 84.91 93.55) (width 0.25) (layer "B.Cu") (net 11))
 (segment (start 84.86 97.56) (end 84.86 93.6) (width 0.25) (layer "B.Cu") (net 11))
 (segment (start 72.66 100.69) (end 74.75 98.6) (width 0.25) (layer "F.Cu") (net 12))
 (segment (start 96.065 97.725) (end 99.885 97.725) (width 0.25) (layer "F.Cu") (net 12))
 (segment (start 99.885 97.725) (end 102.47 95.14) (width 0.25) (layer "F.Cu") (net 12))
 (segment (start 74.75 98.6) (end 95.19 98.6) (width 0.25) (layer "F.Cu") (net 12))
 (segment (start 95.19 98.6) (end 96.065 97.725) (width 0.25) (layer "F.Cu") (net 12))
 (segment (start 75.625 100.265) (end 99.885 100.265) (width 0.25) (layer "F.Cu") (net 13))
 (segment (start 99.885 100.265) (end 102.47 97.68) (width 0.25) (layer "F.Cu") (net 13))
 (segment (start 72.66 103.23) (end 75.625 100.265) (width 0.25) (layer "F.Cu") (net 13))
 (segment (start 81.625 86.995) (end 81.54 87.08) (width 0.25) (layer "F.Cu") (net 14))
 (segment (start 82.7 86.995) (end 81.625 86.995) (width 0.25) (layer "F.Cu") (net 14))
 (via (at 81.54 87.08) (size 0.8) (drill 0.4) (layers "F.Cu" "B.Cu") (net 14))
 (via (at 81.445 90.48) (size 0.8) (drill 0.4) (layers "F.Cu" "B.Cu") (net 14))
 (segment (start 81.445 87.175) (end 81.445 90.48) (width 0.25) (layer "B.Cu") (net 14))
 (segment (start 81.54 87.08) (end 81.445 87.175) (width 0.25) (layer "B.Cu") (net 14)))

